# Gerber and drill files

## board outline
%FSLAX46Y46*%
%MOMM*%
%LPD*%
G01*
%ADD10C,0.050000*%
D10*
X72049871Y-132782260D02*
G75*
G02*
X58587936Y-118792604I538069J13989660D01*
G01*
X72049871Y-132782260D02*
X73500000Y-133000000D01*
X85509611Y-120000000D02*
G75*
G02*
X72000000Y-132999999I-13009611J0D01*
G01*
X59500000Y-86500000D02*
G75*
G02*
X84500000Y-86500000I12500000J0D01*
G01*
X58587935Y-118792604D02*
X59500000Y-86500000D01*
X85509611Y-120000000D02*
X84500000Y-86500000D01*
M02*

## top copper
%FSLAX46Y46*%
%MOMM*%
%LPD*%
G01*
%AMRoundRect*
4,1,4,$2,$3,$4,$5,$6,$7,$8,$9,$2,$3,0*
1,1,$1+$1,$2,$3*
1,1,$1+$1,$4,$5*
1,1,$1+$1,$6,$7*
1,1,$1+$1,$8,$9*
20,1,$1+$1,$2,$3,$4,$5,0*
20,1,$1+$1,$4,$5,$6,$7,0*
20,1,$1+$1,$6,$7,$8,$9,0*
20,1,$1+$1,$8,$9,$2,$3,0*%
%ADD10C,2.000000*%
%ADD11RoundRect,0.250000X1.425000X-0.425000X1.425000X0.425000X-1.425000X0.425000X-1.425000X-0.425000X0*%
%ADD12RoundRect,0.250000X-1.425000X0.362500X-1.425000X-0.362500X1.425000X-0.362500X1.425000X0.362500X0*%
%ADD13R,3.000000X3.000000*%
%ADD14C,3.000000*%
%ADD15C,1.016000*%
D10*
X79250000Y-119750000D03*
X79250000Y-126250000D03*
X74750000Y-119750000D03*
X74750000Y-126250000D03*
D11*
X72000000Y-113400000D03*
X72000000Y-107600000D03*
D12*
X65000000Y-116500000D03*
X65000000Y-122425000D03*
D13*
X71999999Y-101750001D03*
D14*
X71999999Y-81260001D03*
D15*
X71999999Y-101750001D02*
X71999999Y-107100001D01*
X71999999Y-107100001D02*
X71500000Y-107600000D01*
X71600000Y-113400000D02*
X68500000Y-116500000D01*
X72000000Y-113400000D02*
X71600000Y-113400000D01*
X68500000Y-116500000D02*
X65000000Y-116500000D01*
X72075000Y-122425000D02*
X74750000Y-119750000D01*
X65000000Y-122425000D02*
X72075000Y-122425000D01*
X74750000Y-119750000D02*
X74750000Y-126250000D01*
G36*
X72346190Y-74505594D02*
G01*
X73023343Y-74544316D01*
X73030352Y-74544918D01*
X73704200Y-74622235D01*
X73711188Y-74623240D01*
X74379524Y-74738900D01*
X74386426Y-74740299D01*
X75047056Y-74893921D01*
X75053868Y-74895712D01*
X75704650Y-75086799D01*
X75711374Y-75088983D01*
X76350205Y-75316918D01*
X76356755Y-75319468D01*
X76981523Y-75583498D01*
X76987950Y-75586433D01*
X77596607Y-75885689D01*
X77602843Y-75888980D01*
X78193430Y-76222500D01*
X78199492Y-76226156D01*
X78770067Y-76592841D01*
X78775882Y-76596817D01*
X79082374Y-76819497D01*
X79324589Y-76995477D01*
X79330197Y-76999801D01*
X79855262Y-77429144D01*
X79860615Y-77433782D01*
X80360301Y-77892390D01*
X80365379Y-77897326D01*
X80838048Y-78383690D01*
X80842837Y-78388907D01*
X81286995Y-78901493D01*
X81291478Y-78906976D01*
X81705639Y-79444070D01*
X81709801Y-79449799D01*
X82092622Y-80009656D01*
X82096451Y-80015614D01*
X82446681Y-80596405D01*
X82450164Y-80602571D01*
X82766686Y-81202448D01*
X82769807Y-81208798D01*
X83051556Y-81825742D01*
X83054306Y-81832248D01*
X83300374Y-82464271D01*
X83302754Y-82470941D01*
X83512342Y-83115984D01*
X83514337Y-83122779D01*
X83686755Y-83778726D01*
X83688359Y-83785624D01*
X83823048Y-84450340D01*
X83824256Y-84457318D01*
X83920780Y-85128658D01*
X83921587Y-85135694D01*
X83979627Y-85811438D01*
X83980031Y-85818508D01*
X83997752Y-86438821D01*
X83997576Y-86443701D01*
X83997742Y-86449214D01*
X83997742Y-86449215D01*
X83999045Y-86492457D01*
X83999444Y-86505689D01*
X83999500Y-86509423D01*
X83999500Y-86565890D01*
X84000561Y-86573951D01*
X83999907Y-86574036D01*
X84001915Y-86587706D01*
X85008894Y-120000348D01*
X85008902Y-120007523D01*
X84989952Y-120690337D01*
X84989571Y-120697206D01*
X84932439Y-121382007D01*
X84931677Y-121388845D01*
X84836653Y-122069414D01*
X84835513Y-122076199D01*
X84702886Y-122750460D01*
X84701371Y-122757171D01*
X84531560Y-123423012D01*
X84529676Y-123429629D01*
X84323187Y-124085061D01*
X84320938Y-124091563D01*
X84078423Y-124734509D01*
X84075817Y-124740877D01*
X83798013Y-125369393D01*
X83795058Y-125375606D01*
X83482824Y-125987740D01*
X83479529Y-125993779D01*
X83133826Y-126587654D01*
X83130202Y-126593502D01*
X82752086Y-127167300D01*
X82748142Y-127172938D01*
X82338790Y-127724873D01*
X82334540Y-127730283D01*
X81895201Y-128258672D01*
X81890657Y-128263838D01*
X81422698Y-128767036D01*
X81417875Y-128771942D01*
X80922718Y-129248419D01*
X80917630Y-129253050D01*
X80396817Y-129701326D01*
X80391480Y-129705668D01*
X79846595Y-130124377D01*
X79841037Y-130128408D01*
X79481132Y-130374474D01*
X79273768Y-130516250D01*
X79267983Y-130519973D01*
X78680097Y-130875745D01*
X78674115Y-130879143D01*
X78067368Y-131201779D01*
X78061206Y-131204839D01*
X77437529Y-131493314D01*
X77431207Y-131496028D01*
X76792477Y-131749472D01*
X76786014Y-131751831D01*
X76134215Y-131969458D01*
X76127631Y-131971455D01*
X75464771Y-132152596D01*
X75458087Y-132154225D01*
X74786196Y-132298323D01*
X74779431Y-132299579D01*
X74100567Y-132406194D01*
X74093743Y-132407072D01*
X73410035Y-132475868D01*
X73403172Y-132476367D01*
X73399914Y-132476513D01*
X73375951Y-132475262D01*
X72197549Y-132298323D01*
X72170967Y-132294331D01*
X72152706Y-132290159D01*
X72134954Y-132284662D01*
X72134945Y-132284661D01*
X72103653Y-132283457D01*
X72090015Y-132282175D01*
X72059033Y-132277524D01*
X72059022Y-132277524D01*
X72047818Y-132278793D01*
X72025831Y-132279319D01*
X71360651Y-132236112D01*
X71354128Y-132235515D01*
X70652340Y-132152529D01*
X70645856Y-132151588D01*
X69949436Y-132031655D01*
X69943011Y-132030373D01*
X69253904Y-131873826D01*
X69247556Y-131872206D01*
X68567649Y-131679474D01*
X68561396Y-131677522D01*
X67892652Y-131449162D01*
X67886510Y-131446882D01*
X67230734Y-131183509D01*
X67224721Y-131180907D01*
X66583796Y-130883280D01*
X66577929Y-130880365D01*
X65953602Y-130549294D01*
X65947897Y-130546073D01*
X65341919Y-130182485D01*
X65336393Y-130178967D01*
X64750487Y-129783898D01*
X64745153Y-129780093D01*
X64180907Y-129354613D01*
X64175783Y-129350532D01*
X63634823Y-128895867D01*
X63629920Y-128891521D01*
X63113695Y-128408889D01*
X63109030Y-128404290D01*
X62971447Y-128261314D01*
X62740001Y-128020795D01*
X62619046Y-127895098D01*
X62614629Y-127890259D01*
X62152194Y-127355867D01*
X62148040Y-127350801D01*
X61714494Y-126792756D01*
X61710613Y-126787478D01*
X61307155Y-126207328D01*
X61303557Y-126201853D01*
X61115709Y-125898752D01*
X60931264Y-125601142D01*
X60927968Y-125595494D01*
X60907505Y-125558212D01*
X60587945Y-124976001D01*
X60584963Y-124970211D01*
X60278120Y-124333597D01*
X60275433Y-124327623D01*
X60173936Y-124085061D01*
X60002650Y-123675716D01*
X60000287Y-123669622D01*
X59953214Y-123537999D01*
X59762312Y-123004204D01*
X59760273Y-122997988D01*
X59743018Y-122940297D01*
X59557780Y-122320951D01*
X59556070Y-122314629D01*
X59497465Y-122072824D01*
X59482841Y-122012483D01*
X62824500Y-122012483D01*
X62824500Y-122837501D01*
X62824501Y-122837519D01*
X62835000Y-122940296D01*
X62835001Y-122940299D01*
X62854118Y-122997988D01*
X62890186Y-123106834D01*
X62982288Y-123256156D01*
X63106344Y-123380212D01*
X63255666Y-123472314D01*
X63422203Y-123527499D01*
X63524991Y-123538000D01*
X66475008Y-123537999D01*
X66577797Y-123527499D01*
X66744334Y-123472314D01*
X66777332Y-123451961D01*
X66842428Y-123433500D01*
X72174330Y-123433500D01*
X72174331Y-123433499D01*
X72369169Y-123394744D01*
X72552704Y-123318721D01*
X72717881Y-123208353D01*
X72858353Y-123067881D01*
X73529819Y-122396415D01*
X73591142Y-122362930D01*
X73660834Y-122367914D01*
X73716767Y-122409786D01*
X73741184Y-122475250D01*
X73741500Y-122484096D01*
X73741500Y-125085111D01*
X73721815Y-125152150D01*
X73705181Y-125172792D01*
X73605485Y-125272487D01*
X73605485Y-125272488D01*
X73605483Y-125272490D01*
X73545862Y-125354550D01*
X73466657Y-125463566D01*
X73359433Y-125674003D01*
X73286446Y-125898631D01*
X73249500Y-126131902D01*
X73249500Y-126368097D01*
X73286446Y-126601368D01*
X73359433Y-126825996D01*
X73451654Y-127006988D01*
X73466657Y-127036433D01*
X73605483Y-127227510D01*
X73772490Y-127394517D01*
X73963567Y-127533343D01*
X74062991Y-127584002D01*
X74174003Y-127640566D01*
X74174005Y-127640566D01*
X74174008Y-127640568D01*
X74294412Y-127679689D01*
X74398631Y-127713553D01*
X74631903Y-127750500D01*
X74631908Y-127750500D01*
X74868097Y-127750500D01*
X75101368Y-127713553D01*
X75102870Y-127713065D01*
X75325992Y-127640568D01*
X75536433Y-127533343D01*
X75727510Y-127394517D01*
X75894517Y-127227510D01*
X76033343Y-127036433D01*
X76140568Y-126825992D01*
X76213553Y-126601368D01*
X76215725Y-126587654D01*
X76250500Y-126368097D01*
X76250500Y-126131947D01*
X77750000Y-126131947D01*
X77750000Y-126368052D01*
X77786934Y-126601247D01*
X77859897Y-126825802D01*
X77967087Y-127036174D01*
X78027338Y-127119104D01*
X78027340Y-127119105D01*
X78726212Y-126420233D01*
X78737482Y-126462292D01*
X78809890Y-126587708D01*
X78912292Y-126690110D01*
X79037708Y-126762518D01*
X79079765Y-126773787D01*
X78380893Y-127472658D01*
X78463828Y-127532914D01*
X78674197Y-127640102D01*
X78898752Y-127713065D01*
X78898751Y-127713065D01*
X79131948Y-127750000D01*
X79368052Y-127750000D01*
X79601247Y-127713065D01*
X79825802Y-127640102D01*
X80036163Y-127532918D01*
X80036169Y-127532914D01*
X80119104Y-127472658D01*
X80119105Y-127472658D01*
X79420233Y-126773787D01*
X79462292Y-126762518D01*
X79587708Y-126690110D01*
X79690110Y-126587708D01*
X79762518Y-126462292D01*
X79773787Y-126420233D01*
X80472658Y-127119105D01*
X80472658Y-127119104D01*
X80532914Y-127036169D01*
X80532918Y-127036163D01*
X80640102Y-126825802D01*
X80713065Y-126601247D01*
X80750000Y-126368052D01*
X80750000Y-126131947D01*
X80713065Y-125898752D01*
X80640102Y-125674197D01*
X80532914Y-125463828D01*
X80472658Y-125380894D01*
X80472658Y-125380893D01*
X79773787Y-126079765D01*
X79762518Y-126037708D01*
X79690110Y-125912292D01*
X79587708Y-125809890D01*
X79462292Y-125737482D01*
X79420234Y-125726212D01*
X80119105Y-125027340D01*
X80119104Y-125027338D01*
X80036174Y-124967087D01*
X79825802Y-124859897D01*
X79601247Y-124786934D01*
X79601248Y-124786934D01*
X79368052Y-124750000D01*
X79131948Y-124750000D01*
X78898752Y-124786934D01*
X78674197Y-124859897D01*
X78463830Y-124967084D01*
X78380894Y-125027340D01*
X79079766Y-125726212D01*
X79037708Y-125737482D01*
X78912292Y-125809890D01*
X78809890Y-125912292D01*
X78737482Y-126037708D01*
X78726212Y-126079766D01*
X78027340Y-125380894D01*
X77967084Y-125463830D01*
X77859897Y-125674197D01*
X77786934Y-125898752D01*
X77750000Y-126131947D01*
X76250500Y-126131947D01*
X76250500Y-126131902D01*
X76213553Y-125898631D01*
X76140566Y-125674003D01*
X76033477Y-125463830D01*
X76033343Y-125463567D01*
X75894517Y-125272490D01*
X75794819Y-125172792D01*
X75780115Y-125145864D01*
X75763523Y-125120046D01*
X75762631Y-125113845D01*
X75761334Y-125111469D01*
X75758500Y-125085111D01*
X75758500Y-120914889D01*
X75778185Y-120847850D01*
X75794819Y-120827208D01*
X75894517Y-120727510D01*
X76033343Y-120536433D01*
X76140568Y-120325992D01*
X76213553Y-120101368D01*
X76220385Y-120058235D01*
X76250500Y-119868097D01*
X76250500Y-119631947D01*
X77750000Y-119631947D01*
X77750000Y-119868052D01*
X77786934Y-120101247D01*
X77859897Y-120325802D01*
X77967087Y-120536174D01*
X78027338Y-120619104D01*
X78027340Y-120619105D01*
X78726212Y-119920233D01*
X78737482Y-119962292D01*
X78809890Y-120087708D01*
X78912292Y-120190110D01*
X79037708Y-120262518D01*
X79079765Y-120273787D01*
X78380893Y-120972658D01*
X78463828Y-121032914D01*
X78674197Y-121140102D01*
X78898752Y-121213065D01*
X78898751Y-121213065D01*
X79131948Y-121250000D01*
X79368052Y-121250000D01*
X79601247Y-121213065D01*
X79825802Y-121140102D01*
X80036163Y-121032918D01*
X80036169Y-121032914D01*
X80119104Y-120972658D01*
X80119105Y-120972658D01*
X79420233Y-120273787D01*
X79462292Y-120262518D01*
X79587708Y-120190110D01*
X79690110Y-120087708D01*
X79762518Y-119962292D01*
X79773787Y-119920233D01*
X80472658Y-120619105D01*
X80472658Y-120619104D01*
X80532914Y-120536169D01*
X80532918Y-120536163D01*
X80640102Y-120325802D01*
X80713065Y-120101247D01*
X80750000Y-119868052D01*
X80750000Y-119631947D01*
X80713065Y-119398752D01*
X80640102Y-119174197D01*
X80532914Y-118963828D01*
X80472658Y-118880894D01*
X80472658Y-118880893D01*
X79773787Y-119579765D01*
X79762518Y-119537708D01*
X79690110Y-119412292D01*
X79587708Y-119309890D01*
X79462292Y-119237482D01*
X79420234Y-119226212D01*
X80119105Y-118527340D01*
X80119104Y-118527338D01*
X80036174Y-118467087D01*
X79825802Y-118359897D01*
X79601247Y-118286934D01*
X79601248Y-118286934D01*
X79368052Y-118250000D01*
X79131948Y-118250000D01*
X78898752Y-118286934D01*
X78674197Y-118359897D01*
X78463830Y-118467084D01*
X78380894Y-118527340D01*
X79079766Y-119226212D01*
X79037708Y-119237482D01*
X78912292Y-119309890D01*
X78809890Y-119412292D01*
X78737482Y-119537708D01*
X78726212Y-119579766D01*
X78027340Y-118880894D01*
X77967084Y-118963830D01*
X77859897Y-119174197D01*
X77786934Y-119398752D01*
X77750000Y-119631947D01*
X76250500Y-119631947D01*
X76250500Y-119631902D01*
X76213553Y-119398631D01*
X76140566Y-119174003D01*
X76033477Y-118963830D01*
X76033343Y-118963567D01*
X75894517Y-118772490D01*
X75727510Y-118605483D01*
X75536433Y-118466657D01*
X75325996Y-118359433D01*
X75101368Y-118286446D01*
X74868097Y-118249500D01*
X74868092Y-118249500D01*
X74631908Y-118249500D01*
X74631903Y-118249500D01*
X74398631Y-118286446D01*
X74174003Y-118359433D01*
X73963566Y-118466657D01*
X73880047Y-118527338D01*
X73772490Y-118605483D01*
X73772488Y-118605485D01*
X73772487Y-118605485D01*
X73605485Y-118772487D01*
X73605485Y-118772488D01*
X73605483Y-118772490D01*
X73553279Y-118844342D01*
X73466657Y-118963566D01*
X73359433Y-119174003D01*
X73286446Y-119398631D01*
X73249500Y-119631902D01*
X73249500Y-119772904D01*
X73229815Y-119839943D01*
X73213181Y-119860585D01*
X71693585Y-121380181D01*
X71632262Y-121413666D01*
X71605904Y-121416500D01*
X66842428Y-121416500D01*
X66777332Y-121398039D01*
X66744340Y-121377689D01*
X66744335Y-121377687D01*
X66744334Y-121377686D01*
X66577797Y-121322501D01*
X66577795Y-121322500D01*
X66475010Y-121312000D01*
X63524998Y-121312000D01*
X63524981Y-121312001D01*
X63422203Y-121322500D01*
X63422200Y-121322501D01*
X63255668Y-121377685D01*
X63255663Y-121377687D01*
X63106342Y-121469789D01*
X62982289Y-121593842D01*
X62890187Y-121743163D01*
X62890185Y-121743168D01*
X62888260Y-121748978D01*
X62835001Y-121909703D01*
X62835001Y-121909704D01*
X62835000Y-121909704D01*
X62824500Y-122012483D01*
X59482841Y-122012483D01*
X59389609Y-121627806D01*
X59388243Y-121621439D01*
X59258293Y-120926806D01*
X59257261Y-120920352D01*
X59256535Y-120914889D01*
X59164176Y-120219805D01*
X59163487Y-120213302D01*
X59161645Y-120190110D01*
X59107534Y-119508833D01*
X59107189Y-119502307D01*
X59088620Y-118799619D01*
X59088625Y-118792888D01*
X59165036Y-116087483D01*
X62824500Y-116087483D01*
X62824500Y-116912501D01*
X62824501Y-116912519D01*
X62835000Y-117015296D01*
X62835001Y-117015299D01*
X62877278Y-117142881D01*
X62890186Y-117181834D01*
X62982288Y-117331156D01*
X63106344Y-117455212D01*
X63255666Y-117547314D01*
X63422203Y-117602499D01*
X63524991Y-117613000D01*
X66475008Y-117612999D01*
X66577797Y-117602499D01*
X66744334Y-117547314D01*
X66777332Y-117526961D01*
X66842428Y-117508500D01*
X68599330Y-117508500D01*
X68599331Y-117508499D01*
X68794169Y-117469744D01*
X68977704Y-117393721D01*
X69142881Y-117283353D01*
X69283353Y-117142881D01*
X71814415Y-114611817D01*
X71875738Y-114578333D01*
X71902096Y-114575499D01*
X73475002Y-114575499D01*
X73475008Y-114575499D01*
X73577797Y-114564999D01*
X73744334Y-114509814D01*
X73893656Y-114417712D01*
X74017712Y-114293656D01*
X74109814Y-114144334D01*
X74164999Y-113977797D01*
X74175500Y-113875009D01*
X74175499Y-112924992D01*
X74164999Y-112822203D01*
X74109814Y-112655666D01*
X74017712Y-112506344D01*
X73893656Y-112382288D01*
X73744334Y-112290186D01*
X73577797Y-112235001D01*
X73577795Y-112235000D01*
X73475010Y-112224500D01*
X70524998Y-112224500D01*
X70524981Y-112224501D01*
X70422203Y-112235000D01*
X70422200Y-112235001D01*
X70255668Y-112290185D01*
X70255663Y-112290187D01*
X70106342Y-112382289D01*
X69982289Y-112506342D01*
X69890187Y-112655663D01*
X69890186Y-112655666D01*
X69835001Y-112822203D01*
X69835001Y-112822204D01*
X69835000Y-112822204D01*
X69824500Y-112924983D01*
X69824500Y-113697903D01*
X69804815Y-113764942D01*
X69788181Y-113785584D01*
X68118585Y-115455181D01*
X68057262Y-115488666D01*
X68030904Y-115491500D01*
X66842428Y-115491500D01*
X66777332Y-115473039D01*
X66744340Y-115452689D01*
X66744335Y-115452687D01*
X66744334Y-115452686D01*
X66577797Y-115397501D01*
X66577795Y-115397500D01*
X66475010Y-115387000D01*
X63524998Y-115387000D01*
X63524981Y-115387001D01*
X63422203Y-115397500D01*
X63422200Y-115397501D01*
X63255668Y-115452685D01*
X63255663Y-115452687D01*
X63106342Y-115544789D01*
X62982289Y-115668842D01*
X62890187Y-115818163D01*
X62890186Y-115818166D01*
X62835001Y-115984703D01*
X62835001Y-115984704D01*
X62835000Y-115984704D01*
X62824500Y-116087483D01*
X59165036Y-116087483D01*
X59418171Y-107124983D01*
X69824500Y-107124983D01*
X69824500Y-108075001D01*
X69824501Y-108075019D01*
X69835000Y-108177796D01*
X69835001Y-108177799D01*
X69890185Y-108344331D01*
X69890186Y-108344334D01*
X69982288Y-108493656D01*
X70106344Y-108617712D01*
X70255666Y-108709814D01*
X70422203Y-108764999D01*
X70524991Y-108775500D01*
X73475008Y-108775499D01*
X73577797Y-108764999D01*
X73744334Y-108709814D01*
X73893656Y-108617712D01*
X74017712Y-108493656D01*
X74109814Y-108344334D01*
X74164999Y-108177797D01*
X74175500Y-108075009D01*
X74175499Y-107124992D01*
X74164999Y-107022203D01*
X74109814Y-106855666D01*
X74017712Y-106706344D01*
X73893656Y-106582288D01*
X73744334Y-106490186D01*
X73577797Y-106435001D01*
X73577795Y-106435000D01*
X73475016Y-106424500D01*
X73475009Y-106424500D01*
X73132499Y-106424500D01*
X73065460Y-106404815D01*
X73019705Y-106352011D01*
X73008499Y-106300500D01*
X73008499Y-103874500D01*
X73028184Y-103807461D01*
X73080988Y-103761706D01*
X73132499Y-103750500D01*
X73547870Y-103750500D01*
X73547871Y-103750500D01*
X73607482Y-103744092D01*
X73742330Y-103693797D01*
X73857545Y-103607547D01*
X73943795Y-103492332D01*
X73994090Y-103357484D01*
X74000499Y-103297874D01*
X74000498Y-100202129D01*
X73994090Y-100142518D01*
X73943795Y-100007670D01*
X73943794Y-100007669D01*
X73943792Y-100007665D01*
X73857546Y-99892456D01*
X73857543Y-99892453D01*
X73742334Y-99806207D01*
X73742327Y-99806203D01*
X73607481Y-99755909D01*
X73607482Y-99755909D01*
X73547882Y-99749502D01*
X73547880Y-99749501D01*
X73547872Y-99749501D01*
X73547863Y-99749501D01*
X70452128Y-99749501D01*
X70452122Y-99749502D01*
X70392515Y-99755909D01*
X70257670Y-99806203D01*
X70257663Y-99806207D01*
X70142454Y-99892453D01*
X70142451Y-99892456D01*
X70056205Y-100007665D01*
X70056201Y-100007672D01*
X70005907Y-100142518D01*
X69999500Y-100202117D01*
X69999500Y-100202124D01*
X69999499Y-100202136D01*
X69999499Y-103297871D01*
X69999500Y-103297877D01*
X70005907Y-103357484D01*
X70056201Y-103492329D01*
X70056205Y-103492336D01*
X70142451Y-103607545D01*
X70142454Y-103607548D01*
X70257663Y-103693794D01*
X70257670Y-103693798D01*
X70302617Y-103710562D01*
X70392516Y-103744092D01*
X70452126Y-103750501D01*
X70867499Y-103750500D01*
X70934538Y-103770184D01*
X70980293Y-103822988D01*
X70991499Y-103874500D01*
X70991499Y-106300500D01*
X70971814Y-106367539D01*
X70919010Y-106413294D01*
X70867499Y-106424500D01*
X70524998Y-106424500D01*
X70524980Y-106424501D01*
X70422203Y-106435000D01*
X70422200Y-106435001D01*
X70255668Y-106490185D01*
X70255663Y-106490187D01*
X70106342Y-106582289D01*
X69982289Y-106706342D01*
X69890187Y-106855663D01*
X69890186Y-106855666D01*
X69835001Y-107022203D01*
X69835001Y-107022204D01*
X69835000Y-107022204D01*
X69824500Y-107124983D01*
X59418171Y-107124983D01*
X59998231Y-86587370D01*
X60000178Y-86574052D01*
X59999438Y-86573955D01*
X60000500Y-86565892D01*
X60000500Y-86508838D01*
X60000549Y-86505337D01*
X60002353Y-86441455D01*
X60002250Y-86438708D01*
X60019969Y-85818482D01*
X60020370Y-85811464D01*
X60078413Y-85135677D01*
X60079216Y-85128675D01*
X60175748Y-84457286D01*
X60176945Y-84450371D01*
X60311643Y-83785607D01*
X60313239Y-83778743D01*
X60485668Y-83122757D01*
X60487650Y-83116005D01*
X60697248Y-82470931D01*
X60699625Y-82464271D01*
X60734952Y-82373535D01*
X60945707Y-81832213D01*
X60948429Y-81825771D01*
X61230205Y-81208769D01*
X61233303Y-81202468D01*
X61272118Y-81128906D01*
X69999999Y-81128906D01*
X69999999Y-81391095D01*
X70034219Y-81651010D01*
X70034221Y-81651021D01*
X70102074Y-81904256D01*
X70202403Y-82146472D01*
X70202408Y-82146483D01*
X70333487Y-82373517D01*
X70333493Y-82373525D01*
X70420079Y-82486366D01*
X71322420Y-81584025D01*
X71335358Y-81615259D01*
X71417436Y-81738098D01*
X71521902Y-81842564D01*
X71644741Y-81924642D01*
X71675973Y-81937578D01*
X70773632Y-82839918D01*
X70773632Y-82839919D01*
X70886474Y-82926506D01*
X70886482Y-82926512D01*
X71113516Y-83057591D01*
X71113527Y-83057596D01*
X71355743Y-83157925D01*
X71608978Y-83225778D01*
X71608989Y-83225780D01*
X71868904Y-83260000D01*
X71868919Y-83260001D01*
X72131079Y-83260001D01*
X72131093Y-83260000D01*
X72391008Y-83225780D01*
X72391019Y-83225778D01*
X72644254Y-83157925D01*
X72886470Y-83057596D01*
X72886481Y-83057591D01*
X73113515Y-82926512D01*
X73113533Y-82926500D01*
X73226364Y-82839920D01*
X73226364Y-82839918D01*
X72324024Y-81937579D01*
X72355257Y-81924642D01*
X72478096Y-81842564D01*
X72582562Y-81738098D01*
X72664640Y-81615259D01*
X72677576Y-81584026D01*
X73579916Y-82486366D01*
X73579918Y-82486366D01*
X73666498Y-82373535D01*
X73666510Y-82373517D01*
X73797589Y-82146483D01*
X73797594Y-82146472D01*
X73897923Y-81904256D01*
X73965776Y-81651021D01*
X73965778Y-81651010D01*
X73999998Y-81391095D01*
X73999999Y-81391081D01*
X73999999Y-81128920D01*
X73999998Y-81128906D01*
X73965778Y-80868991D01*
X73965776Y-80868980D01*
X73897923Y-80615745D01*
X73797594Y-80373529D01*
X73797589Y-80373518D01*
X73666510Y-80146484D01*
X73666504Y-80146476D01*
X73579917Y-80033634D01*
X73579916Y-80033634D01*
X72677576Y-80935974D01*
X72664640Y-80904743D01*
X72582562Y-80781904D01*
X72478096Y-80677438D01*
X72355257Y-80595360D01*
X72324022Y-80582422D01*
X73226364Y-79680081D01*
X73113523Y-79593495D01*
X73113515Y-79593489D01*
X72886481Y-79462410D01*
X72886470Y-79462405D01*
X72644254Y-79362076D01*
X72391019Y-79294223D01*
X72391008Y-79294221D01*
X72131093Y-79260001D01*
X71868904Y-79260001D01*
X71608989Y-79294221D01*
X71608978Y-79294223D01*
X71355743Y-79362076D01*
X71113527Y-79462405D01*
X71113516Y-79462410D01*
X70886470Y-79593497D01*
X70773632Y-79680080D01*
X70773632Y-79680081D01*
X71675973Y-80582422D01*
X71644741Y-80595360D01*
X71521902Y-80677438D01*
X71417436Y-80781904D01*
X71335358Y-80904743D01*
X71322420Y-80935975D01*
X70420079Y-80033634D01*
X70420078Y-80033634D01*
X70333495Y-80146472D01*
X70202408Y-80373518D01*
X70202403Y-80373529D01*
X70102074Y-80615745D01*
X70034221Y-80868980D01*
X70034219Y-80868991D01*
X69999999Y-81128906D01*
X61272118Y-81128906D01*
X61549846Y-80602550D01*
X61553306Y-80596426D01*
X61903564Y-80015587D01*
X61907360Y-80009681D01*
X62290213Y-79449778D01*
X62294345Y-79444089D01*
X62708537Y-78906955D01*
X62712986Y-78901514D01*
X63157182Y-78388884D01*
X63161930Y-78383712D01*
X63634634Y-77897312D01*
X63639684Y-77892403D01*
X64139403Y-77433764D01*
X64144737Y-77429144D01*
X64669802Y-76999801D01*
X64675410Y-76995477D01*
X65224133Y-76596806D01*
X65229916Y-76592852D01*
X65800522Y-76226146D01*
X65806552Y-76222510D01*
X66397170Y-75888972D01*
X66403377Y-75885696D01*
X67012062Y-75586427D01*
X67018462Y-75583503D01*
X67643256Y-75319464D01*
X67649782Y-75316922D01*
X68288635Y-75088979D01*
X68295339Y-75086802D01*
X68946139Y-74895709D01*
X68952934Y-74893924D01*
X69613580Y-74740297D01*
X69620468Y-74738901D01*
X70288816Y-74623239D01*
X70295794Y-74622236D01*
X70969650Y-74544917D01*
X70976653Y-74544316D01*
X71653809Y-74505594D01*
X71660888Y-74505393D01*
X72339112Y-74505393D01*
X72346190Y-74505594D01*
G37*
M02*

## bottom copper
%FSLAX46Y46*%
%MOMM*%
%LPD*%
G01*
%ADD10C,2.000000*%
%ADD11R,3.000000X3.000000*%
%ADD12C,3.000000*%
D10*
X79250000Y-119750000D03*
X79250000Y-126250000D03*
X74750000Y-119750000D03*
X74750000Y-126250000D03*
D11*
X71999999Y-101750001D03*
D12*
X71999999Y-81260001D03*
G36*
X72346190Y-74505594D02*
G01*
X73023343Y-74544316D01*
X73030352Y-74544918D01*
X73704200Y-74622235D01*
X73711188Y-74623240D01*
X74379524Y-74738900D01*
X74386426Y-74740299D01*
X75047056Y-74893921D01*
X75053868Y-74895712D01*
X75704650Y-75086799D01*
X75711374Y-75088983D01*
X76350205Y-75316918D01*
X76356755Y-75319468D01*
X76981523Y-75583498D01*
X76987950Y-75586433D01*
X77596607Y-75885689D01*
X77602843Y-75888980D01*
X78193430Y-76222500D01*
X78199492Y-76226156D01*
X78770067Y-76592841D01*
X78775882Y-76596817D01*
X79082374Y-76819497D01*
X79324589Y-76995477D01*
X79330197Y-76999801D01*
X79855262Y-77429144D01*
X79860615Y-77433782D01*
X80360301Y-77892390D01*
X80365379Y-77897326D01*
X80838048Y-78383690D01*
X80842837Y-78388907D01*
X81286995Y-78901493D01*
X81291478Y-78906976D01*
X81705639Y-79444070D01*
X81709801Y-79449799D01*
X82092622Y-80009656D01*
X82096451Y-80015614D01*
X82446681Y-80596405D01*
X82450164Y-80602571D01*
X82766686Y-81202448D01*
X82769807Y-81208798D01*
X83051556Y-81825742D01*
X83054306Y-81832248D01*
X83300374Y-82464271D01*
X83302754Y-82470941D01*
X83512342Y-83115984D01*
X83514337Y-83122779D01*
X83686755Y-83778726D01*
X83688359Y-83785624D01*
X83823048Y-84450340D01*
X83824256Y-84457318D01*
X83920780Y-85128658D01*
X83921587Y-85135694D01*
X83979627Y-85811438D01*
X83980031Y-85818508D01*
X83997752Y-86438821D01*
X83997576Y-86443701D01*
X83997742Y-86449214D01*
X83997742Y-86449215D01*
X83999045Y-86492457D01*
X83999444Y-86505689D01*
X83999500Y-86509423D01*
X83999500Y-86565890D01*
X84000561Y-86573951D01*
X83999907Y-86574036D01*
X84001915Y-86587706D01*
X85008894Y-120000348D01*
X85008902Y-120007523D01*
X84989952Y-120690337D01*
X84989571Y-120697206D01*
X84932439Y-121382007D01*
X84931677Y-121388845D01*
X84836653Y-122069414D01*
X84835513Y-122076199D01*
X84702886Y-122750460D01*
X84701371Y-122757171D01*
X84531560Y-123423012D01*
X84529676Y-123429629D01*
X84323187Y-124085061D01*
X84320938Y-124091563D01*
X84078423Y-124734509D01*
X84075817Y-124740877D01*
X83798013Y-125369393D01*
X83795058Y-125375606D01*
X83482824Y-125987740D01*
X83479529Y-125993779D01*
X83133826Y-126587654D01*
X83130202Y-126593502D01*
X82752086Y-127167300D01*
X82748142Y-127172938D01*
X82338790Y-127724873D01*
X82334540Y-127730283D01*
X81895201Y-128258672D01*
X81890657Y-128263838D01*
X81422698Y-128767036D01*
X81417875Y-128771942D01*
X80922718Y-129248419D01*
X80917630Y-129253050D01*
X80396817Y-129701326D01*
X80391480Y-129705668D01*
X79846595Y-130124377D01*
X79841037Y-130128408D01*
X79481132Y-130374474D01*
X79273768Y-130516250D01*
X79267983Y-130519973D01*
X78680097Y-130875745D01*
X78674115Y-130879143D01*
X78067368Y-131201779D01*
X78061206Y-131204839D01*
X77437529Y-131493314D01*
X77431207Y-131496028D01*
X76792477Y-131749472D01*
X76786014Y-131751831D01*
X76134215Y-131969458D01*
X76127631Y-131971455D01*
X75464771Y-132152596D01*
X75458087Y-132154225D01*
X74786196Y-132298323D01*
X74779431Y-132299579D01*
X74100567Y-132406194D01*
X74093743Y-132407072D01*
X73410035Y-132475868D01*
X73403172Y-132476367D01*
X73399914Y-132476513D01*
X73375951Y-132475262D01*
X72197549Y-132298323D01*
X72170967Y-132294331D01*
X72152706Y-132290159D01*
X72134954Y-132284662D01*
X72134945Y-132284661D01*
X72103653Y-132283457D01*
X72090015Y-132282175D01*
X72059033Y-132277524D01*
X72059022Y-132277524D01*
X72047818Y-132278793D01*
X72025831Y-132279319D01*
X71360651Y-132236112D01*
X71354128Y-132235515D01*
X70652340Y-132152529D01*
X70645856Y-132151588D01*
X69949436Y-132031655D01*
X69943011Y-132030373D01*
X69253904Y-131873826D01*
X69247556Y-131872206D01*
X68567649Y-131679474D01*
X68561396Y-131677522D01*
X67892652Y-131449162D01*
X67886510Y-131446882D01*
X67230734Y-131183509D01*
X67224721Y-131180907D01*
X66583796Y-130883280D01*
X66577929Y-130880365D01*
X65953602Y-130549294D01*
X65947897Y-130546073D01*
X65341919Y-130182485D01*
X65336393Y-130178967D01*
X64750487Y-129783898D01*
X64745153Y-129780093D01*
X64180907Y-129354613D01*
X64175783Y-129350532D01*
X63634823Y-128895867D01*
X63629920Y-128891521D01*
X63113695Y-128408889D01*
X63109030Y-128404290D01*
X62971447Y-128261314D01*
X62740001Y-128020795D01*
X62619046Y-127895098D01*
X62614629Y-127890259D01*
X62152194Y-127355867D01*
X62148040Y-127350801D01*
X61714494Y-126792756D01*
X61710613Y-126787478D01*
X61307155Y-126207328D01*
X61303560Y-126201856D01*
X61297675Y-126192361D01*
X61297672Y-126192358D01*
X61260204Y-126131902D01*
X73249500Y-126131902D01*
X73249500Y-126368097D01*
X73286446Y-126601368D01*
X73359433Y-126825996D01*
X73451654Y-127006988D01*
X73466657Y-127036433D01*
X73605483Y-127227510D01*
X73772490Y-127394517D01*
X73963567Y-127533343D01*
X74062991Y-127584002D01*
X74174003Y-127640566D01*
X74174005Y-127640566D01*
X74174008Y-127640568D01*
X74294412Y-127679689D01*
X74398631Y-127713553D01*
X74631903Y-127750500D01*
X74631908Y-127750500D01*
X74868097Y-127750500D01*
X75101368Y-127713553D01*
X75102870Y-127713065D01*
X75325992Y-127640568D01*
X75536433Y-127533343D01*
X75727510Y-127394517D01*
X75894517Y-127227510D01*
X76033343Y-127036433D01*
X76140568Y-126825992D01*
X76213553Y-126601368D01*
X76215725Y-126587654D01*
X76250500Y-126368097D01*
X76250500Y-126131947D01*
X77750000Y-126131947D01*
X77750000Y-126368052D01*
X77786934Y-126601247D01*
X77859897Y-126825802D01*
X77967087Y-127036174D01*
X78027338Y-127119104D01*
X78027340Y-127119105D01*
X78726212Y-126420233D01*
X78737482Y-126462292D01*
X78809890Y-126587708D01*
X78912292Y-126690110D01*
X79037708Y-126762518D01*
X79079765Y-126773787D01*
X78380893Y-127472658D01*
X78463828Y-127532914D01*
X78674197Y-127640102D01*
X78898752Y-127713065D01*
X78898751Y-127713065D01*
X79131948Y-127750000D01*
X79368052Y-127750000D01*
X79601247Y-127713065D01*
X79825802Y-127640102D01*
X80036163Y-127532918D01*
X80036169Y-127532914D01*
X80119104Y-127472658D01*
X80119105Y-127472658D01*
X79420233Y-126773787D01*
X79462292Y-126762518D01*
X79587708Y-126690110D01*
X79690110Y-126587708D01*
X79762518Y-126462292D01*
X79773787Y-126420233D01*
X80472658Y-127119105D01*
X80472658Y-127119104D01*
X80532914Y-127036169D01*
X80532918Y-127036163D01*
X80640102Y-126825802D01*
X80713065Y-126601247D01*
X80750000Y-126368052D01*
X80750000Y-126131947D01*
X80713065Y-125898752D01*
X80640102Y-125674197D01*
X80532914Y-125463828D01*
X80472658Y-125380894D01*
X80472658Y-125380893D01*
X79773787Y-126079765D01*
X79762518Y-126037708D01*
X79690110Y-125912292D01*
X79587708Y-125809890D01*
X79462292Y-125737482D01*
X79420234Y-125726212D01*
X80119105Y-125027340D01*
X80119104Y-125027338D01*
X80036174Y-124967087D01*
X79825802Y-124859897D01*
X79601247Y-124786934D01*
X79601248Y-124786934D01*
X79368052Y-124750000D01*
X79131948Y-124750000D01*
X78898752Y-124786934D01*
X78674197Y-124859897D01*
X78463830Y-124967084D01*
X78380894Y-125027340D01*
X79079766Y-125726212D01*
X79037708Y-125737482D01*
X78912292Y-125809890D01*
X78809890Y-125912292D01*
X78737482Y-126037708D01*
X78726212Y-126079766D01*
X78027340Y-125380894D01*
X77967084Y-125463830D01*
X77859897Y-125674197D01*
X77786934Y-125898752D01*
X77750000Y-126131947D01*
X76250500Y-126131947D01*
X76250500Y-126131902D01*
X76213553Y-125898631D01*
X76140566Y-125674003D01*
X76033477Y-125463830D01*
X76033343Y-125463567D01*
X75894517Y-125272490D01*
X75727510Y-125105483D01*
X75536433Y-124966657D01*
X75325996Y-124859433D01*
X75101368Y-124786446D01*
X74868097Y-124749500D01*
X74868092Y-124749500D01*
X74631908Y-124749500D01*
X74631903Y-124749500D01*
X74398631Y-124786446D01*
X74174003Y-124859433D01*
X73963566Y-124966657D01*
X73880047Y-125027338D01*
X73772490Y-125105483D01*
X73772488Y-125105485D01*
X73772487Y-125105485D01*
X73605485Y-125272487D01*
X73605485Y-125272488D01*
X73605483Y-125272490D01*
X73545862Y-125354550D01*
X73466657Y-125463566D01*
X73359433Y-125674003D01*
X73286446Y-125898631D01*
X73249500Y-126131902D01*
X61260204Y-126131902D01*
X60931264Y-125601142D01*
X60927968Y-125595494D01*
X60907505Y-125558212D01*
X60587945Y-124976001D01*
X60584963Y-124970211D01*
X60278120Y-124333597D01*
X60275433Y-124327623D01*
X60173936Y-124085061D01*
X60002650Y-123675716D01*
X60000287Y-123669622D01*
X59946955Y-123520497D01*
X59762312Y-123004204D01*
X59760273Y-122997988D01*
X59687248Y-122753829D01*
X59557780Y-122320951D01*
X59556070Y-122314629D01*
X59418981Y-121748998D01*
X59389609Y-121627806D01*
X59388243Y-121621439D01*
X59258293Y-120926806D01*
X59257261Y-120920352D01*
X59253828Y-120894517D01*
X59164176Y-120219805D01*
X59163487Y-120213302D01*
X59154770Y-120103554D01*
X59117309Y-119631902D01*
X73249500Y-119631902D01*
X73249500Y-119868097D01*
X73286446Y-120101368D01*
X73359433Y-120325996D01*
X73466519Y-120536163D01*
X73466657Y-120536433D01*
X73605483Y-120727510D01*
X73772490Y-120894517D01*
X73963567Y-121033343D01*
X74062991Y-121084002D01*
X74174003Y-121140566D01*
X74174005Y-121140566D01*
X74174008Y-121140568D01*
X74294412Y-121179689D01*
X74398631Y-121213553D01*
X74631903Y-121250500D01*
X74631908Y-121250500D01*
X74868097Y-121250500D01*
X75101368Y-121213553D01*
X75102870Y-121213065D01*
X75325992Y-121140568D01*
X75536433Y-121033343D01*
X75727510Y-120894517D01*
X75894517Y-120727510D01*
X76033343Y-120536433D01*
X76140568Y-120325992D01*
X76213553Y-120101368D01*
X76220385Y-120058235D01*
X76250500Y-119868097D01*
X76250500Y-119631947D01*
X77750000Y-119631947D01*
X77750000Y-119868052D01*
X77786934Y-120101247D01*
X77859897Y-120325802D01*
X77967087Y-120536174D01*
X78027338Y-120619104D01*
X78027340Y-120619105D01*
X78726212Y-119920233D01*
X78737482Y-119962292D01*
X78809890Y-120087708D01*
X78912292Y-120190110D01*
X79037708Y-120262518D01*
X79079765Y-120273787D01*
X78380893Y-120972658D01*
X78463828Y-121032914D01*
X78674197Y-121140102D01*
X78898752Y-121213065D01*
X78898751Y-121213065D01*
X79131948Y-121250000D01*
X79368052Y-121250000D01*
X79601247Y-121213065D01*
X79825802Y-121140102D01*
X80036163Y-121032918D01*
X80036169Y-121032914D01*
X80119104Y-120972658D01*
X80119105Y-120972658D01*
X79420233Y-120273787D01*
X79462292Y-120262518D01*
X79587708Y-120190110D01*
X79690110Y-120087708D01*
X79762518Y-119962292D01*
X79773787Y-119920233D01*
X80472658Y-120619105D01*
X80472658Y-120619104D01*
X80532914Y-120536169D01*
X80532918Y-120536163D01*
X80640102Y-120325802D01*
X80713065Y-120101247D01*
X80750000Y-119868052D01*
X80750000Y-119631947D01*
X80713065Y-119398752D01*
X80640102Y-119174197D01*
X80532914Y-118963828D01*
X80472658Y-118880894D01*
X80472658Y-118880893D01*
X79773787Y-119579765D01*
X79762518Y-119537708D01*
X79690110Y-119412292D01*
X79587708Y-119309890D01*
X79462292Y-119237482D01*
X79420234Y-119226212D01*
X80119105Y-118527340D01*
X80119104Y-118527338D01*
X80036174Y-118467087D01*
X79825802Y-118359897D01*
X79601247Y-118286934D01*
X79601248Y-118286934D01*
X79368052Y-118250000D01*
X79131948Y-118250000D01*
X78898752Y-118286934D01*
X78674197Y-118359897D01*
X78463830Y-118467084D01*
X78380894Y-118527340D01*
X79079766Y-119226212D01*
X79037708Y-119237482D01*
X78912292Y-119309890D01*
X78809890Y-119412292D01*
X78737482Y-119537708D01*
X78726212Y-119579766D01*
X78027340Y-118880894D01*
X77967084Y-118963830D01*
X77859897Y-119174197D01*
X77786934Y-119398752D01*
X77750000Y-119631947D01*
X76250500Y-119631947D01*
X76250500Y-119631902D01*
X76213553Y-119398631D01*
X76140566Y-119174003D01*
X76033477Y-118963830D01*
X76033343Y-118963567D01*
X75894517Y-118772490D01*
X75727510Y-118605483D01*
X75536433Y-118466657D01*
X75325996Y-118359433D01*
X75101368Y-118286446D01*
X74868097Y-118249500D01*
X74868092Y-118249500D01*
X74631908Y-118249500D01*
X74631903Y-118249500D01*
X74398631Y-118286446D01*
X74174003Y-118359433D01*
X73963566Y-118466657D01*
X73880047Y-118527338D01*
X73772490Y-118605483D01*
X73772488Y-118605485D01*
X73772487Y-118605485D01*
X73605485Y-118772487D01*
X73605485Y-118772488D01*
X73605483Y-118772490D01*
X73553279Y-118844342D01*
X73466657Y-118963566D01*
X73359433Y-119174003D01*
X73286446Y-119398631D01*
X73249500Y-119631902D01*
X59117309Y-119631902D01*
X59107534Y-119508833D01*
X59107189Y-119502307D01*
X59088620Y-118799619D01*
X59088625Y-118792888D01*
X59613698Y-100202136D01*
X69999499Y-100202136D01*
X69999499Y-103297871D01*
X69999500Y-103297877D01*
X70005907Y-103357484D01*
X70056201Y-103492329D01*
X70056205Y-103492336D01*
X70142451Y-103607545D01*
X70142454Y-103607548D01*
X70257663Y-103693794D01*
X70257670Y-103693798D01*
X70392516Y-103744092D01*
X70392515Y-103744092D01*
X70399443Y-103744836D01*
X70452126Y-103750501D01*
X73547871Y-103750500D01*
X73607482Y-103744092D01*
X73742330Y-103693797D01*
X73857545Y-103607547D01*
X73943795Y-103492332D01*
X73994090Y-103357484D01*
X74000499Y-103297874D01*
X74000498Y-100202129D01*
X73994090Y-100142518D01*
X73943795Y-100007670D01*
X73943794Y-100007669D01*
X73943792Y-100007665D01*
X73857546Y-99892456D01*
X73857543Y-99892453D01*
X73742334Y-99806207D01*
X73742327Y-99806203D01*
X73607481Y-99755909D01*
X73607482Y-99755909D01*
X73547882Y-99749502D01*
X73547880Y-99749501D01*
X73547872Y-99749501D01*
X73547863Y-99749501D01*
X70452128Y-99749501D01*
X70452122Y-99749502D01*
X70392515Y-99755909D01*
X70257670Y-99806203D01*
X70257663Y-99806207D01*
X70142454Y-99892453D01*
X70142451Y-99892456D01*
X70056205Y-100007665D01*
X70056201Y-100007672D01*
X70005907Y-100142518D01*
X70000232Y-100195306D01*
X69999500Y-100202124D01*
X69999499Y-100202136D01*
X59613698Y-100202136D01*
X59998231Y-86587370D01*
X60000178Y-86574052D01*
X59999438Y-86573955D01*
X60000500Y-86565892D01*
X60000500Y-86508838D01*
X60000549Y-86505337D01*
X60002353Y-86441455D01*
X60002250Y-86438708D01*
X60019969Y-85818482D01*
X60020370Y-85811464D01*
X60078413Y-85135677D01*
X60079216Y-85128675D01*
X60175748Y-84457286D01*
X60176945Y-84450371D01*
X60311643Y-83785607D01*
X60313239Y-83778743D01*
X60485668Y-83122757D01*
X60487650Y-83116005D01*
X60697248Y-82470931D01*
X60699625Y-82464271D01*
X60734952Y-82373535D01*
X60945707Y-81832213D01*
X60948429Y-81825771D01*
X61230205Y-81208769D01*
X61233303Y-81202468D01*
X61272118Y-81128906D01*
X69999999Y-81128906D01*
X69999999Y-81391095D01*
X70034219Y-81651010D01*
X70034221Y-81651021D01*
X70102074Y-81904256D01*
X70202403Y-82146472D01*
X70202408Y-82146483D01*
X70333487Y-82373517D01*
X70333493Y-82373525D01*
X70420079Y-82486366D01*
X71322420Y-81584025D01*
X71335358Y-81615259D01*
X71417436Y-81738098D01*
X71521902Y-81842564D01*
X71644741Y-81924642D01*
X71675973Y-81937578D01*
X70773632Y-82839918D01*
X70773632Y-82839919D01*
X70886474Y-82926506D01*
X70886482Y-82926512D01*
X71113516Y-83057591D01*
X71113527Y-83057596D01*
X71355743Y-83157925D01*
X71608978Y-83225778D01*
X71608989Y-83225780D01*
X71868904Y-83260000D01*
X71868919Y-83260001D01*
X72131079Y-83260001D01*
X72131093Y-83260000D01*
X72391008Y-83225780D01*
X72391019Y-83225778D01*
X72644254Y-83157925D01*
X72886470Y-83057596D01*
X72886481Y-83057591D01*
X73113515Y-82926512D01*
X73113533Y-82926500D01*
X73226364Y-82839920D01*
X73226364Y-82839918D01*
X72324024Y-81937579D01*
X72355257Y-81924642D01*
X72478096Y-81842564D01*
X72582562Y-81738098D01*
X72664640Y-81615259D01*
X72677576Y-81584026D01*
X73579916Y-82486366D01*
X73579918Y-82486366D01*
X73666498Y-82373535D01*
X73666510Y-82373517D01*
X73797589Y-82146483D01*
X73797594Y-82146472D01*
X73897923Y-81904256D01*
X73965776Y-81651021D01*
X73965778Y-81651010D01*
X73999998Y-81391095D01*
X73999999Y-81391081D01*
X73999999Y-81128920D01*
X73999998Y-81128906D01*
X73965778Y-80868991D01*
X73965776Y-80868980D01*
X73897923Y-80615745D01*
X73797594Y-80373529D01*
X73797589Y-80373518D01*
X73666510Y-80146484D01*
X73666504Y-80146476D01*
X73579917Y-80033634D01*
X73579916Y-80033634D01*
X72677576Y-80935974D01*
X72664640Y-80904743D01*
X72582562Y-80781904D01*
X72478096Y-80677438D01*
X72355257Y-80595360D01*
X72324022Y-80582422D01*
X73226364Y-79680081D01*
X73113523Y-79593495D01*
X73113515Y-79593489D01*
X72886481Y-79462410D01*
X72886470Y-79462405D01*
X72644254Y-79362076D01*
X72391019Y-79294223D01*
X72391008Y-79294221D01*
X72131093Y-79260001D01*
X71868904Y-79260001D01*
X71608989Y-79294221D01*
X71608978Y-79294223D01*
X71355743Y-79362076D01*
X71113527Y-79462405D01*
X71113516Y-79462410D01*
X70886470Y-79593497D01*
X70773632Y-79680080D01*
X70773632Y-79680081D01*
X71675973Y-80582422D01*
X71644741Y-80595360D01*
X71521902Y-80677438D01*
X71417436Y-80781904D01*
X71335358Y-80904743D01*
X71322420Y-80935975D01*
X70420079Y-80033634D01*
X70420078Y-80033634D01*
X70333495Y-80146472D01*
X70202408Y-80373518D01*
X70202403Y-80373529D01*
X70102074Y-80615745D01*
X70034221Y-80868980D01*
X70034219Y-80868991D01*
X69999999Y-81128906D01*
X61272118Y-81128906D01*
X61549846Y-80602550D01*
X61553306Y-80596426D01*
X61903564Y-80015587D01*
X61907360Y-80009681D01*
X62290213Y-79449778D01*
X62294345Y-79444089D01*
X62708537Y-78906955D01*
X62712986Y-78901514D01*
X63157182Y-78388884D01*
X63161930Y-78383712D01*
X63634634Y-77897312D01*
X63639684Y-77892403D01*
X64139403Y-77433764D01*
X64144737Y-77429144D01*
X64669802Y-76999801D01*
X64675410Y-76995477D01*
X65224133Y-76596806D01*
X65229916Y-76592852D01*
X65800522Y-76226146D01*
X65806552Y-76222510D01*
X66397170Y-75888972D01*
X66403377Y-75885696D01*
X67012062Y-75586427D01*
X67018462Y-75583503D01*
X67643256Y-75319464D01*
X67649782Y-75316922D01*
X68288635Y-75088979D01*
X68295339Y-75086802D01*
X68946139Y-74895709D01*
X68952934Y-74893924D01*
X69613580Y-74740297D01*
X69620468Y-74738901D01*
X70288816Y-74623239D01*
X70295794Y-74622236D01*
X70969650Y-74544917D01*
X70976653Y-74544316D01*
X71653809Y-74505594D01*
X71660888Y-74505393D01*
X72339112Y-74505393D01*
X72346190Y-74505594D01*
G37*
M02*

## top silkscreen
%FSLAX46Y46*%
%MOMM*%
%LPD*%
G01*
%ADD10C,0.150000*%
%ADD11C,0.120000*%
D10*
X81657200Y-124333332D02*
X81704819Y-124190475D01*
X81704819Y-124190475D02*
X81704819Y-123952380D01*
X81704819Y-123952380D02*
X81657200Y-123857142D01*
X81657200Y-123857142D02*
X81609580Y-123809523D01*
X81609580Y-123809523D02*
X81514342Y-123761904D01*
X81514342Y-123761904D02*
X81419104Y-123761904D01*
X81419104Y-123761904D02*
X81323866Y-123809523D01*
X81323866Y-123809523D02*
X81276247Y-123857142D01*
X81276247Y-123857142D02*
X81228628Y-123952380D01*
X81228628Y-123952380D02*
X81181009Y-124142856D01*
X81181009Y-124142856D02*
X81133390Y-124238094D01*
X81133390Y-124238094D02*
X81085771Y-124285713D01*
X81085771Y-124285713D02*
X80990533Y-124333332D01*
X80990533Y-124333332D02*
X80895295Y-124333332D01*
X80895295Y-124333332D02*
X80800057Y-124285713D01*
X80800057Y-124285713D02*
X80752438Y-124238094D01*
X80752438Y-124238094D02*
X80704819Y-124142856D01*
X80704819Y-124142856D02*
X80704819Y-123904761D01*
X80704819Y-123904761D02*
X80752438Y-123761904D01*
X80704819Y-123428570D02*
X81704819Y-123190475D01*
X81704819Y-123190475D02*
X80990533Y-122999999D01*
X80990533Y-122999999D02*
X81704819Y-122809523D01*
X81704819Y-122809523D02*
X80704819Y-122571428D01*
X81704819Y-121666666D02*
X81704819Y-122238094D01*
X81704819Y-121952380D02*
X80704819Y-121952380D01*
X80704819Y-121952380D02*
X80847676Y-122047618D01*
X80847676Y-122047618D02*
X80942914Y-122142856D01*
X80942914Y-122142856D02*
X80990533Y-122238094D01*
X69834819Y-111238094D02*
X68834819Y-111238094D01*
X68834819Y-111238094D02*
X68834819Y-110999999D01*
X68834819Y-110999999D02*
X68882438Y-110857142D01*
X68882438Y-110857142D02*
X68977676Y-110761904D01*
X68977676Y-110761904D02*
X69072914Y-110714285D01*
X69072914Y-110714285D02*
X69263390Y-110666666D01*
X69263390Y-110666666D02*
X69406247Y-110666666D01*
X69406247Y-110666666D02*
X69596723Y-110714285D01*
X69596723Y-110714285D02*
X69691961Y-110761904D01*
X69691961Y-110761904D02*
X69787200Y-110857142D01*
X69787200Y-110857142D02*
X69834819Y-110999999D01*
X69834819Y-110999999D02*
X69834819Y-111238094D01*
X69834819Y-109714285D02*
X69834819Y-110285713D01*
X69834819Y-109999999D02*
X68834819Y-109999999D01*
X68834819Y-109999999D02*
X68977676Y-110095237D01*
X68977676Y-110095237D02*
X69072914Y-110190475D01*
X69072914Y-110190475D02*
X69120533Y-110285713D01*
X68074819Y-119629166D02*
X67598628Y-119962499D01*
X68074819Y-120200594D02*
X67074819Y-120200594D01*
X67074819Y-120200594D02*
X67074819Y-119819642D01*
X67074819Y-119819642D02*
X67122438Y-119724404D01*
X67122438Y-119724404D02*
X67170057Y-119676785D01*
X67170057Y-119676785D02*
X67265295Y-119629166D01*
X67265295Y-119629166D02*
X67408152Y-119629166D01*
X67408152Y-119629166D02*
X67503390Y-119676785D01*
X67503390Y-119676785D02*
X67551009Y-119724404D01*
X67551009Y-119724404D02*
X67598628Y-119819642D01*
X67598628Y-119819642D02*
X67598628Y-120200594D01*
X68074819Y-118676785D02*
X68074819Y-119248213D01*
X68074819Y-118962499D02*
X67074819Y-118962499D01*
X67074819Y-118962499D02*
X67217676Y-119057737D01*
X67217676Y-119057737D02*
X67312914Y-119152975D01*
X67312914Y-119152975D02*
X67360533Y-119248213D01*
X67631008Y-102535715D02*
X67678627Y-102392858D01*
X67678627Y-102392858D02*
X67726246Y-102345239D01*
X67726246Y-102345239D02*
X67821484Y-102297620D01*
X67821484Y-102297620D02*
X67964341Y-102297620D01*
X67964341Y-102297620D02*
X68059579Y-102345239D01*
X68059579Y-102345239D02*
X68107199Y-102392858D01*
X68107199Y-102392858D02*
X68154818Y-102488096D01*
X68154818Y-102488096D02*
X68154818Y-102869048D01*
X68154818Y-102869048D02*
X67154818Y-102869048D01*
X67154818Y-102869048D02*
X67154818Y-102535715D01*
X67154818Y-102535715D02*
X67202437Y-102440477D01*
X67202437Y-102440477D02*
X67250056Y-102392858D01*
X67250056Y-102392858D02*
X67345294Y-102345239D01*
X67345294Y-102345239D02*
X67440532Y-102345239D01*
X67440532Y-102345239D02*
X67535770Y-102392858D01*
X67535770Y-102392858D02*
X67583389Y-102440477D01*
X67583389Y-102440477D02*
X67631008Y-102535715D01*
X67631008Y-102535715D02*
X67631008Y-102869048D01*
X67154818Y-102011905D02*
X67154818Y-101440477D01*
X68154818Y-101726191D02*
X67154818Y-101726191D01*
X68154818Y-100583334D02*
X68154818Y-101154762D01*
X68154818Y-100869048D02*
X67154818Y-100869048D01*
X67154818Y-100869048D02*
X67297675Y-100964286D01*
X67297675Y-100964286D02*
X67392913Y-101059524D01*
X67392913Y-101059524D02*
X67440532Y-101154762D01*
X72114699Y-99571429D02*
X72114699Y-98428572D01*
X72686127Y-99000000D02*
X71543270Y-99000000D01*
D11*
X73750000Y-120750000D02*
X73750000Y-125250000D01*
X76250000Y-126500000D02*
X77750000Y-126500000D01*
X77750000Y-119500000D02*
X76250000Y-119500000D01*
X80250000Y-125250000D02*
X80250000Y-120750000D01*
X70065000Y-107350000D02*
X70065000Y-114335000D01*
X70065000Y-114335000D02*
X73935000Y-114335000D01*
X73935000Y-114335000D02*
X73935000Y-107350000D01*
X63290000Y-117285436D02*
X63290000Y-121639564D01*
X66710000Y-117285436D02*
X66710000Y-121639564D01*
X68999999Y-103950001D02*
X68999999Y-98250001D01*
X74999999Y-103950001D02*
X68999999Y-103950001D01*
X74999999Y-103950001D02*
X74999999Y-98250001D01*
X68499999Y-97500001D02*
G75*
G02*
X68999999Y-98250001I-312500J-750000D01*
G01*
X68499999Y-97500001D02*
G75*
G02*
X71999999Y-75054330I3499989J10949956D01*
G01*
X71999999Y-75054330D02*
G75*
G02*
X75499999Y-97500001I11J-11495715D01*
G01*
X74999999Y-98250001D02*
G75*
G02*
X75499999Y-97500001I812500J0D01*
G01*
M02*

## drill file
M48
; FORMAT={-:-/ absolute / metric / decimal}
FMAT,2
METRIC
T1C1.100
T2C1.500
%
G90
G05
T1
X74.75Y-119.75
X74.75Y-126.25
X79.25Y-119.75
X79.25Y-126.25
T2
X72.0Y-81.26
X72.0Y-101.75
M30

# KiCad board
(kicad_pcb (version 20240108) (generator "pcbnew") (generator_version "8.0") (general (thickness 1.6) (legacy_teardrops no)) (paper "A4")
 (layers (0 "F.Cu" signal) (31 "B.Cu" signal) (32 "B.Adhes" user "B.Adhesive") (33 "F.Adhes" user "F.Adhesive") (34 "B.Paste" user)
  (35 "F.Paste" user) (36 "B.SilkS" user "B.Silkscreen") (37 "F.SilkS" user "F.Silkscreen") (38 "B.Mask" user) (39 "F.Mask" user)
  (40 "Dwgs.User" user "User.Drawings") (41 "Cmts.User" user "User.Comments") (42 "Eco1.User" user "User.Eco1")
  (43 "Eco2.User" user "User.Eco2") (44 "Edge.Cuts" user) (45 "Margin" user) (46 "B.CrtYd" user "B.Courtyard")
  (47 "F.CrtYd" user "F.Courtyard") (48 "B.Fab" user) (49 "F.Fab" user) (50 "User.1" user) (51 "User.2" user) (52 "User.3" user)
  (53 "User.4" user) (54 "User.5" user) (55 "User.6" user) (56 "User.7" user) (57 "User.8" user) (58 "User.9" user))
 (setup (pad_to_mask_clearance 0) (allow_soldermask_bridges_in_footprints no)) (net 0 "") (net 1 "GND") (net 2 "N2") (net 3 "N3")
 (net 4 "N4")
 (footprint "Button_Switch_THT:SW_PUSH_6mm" (layer "F.Cu") (at 79.25 119.75 -90)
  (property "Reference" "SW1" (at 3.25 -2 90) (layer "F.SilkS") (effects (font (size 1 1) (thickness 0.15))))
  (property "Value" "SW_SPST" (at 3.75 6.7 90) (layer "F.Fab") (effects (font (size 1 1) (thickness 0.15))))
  (fp_line (start 1 5.5) (end 5.5 5.5) (stroke (width 0.12) (type solid)) (layer "F.SilkS"))
  (fp_line (start 6.75 3) (end 6.75 1.5) (stroke (width 0.12) (type solid)) (layer "F.SilkS"))
  (fp_line (start -0.25 1.5) (end -0.25 3) (stroke (width 0.12) (type solid)) (layer "F.SilkS"))
  (fp_line (start 5.5 -1) (end 1 -1) (stroke (width 0.12) (type solid)) (layer "F.SilkS"))
  (pad "1" thru_hole circle (at 0 0) (size 2 2) (drill 1.1) (layers "*.Cu" "*.Mask") (remove_unused_layers no) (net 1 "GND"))
  (pad "1" thru_hole circle (at 6.5 0) (size 2 2) (drill 1.1) (layers "*.Cu" "*.Mask") (remove_unused_layers no) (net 1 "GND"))
  (pad "2" thru_hole circle (at 0 4.5) (size 2 2) (drill 1.1) (layers "*.Cu" "*.Mask") (remove_unused_layers no) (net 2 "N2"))
  (pad "2" thru_hole circle (at 6.5 4.5) (size 2 2) (drill 1.1) (layers "*.Cu" "*.Mask") (remove_unused_layers no) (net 2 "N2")))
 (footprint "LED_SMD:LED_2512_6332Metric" (layer "F.Cu") (at 72 110.5 90)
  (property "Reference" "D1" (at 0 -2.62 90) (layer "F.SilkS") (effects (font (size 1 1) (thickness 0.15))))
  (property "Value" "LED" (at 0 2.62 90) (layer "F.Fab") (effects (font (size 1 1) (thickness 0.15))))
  (fp_line (start 3.15 -1.935) (end -3.835 -1.935) (stroke (width 0.12) (type solid)) (layer "F.SilkS"))
  (fp_line (start -3.835 -1.935) (end -3.835 1.935) (stroke (width 0.12) (type solid)) (layer "F.SilkS"))
  (fp_line (start -3.835 1.935) (end 3.15 1.935) (stroke (width 0.12) (type solid)) (layer "F.SilkS"))
  (pad "1" smd roundrect (at -2.9 0 90) (size 1.35 3.35) (layers "F.Cu" "F.Paste" "F.Mask") (roundrect_rratio 0.185185) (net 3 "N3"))
  (pad "2" smd roundrect (at 2.9 0 90) (size 1.35 3.35) (layers "F.Cu" "F.Paste" "F.Mask") (roundrect_rratio 0.185185) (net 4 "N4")))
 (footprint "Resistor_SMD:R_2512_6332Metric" (layer "F.Cu") (at 65 119.4625 -90)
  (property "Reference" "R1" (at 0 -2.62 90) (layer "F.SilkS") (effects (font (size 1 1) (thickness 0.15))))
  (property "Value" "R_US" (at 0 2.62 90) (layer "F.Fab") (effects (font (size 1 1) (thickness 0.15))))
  (fp_line (start -2.177064 1.71) (end 2.177064 1.71) (stroke (width 0.12) (type solid)) (layer "F.SilkS"))
  (fp_line (start -2.177064 -1.71) (end 2.177064 -1.71) (stroke (width 0.12) (type solid)) (layer "F.SilkS"))
  (pad "1" smd roundrect (at -2.9625 0 270) (size 1.225 3.35) (layers "F.Cu" "F.Paste" "F.Mask") (roundrect_rratio 0.204082) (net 3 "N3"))
  (pad "2" smd roundrect (at 2.9625 0 270) (size 1.225 3.35) (layers "F.Cu" "F.Paste" "F.Mask") (roundrect_rratio 0.204082) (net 2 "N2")))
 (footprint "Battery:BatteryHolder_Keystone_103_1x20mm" (layer "F.Cu") (at 71.999999 101.750001 90)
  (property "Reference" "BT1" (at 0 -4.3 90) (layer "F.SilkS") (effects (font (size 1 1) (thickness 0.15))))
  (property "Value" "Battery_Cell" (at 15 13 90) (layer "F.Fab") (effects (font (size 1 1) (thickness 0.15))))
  (fp_line (start -2.2 -3) (end 3.5 -3) (stroke (width 0.12) (type solid)) (layer "F.SilkS"))
  (fp_line (start -2.2 3) (end -2.2 -3) (stroke (width 0.12) (type solid)) (layer "F.SilkS"))
  (fp_line (start -2.2 3) (end 3.5 3) (stroke (width 0.12) (type solid)) (layer "F.SilkS"))
  (fp_arc (start 4.25 -3.5) (mid 3.950694 -3.136459) (end 3.5 -3) (stroke (width 0.12) (type solid)) (layer "F.SilkS"))
  (fp_arc (start 4.25 -3.5) (mid 16.971103 -11.358466) (end 26.695671 0) (stroke (width 0.12) (type solid)) (layer "F.SilkS"))
  (fp_arc (start 26.695671 0) (mid 16.971103 11.358466) (end 4.25 3.5) (stroke (width 0.12) (type solid)) (layer "F.SilkS"))
  (fp_arc (start 3.5 3) (mid 3.950694 3.136459) (end 4.25 3.5) (stroke (width 0.12) (type solid)) (layer "F.SilkS"))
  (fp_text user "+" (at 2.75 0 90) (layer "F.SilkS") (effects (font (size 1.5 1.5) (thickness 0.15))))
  (pad "1" thru_hole rect (at 0 0 90) (size 3 3) (drill 1.5) (layers "*.Cu" "*.Mask") (remove_unused_layers no) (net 4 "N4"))
  (pad "2" thru_hole circle (at 20.49 0 90) (size 3 3) (drill 1.5) (layers "*.Cu" "*.Mask") (remove_unused_layers no) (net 1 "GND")))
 (gr_arc (start 72.049871 132.78226) (mid 62.5 128.5) (end 58.587935 118.792604) (stroke (width 0.05) (type default)) (layer "Edge.Cuts"))
 (gr_line (start 72.049871 132.78226) (end 73.5 133) (stroke (width 0.05) (type default)) (layer "Edge.Cuts"))
 (gr_arc (start 85.509611 120) (mid 81.520675 129.374294) (end 72 132.999999) (stroke (width 0.05) (type default)) (layer "Edge.Cuts"))
 (gr_arc (start 59.5 86.5) (mid 72 74) (end 84.5 86.5) (stroke (width 0.05) (type default)) (layer "Edge.Cuts"))
 (gr_line (start 58.587935 118.792604) (end 59.5 86.5) (stroke (width 0.05) (type default)) (layer "Edge.Cuts"))
 (gr_line (start 85.509611 120) (end 84.5 86.5) (stroke (width 0.05) (type default)) (layer "Edge.Cuts"))
 (segment (start 71.999999 101.750001) (end 71.999999 107.100001) (width 1.016) (layer "F.Cu") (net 4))
 (segment (start 71.999999 107.100001) (end 71.5 107.6) (width 1.016) (layer "F.Cu") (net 4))
 (segment (start 71.6 113.4) (end 68.5 116.5) (width 1.016) (layer "F.Cu") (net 3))
 (segment (start 72 113.4) (end 71.6 113.4) (width 1.016) (layer "F.Cu") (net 3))
 (segment (start 68.5 116.5) (end 65 116.5) (width 1.016) (layer "F.Cu") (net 3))
 (segment (start 72.075 122.425) (end 74.75 119.75) (width 1.016) (layer "F.Cu") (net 2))
 (segment (start 65 122.425) (end 72.075 122.425) (width 1.016) (layer "F.Cu") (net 2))
 (segment (start 74.75 119.75) (end 74.75 126.25) (width 1.016) (layer "F.Cu") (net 2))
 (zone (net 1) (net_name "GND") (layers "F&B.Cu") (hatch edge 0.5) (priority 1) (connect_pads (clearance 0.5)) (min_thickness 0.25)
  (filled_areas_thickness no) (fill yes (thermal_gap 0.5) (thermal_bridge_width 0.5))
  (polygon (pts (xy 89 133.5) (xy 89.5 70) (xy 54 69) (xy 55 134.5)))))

